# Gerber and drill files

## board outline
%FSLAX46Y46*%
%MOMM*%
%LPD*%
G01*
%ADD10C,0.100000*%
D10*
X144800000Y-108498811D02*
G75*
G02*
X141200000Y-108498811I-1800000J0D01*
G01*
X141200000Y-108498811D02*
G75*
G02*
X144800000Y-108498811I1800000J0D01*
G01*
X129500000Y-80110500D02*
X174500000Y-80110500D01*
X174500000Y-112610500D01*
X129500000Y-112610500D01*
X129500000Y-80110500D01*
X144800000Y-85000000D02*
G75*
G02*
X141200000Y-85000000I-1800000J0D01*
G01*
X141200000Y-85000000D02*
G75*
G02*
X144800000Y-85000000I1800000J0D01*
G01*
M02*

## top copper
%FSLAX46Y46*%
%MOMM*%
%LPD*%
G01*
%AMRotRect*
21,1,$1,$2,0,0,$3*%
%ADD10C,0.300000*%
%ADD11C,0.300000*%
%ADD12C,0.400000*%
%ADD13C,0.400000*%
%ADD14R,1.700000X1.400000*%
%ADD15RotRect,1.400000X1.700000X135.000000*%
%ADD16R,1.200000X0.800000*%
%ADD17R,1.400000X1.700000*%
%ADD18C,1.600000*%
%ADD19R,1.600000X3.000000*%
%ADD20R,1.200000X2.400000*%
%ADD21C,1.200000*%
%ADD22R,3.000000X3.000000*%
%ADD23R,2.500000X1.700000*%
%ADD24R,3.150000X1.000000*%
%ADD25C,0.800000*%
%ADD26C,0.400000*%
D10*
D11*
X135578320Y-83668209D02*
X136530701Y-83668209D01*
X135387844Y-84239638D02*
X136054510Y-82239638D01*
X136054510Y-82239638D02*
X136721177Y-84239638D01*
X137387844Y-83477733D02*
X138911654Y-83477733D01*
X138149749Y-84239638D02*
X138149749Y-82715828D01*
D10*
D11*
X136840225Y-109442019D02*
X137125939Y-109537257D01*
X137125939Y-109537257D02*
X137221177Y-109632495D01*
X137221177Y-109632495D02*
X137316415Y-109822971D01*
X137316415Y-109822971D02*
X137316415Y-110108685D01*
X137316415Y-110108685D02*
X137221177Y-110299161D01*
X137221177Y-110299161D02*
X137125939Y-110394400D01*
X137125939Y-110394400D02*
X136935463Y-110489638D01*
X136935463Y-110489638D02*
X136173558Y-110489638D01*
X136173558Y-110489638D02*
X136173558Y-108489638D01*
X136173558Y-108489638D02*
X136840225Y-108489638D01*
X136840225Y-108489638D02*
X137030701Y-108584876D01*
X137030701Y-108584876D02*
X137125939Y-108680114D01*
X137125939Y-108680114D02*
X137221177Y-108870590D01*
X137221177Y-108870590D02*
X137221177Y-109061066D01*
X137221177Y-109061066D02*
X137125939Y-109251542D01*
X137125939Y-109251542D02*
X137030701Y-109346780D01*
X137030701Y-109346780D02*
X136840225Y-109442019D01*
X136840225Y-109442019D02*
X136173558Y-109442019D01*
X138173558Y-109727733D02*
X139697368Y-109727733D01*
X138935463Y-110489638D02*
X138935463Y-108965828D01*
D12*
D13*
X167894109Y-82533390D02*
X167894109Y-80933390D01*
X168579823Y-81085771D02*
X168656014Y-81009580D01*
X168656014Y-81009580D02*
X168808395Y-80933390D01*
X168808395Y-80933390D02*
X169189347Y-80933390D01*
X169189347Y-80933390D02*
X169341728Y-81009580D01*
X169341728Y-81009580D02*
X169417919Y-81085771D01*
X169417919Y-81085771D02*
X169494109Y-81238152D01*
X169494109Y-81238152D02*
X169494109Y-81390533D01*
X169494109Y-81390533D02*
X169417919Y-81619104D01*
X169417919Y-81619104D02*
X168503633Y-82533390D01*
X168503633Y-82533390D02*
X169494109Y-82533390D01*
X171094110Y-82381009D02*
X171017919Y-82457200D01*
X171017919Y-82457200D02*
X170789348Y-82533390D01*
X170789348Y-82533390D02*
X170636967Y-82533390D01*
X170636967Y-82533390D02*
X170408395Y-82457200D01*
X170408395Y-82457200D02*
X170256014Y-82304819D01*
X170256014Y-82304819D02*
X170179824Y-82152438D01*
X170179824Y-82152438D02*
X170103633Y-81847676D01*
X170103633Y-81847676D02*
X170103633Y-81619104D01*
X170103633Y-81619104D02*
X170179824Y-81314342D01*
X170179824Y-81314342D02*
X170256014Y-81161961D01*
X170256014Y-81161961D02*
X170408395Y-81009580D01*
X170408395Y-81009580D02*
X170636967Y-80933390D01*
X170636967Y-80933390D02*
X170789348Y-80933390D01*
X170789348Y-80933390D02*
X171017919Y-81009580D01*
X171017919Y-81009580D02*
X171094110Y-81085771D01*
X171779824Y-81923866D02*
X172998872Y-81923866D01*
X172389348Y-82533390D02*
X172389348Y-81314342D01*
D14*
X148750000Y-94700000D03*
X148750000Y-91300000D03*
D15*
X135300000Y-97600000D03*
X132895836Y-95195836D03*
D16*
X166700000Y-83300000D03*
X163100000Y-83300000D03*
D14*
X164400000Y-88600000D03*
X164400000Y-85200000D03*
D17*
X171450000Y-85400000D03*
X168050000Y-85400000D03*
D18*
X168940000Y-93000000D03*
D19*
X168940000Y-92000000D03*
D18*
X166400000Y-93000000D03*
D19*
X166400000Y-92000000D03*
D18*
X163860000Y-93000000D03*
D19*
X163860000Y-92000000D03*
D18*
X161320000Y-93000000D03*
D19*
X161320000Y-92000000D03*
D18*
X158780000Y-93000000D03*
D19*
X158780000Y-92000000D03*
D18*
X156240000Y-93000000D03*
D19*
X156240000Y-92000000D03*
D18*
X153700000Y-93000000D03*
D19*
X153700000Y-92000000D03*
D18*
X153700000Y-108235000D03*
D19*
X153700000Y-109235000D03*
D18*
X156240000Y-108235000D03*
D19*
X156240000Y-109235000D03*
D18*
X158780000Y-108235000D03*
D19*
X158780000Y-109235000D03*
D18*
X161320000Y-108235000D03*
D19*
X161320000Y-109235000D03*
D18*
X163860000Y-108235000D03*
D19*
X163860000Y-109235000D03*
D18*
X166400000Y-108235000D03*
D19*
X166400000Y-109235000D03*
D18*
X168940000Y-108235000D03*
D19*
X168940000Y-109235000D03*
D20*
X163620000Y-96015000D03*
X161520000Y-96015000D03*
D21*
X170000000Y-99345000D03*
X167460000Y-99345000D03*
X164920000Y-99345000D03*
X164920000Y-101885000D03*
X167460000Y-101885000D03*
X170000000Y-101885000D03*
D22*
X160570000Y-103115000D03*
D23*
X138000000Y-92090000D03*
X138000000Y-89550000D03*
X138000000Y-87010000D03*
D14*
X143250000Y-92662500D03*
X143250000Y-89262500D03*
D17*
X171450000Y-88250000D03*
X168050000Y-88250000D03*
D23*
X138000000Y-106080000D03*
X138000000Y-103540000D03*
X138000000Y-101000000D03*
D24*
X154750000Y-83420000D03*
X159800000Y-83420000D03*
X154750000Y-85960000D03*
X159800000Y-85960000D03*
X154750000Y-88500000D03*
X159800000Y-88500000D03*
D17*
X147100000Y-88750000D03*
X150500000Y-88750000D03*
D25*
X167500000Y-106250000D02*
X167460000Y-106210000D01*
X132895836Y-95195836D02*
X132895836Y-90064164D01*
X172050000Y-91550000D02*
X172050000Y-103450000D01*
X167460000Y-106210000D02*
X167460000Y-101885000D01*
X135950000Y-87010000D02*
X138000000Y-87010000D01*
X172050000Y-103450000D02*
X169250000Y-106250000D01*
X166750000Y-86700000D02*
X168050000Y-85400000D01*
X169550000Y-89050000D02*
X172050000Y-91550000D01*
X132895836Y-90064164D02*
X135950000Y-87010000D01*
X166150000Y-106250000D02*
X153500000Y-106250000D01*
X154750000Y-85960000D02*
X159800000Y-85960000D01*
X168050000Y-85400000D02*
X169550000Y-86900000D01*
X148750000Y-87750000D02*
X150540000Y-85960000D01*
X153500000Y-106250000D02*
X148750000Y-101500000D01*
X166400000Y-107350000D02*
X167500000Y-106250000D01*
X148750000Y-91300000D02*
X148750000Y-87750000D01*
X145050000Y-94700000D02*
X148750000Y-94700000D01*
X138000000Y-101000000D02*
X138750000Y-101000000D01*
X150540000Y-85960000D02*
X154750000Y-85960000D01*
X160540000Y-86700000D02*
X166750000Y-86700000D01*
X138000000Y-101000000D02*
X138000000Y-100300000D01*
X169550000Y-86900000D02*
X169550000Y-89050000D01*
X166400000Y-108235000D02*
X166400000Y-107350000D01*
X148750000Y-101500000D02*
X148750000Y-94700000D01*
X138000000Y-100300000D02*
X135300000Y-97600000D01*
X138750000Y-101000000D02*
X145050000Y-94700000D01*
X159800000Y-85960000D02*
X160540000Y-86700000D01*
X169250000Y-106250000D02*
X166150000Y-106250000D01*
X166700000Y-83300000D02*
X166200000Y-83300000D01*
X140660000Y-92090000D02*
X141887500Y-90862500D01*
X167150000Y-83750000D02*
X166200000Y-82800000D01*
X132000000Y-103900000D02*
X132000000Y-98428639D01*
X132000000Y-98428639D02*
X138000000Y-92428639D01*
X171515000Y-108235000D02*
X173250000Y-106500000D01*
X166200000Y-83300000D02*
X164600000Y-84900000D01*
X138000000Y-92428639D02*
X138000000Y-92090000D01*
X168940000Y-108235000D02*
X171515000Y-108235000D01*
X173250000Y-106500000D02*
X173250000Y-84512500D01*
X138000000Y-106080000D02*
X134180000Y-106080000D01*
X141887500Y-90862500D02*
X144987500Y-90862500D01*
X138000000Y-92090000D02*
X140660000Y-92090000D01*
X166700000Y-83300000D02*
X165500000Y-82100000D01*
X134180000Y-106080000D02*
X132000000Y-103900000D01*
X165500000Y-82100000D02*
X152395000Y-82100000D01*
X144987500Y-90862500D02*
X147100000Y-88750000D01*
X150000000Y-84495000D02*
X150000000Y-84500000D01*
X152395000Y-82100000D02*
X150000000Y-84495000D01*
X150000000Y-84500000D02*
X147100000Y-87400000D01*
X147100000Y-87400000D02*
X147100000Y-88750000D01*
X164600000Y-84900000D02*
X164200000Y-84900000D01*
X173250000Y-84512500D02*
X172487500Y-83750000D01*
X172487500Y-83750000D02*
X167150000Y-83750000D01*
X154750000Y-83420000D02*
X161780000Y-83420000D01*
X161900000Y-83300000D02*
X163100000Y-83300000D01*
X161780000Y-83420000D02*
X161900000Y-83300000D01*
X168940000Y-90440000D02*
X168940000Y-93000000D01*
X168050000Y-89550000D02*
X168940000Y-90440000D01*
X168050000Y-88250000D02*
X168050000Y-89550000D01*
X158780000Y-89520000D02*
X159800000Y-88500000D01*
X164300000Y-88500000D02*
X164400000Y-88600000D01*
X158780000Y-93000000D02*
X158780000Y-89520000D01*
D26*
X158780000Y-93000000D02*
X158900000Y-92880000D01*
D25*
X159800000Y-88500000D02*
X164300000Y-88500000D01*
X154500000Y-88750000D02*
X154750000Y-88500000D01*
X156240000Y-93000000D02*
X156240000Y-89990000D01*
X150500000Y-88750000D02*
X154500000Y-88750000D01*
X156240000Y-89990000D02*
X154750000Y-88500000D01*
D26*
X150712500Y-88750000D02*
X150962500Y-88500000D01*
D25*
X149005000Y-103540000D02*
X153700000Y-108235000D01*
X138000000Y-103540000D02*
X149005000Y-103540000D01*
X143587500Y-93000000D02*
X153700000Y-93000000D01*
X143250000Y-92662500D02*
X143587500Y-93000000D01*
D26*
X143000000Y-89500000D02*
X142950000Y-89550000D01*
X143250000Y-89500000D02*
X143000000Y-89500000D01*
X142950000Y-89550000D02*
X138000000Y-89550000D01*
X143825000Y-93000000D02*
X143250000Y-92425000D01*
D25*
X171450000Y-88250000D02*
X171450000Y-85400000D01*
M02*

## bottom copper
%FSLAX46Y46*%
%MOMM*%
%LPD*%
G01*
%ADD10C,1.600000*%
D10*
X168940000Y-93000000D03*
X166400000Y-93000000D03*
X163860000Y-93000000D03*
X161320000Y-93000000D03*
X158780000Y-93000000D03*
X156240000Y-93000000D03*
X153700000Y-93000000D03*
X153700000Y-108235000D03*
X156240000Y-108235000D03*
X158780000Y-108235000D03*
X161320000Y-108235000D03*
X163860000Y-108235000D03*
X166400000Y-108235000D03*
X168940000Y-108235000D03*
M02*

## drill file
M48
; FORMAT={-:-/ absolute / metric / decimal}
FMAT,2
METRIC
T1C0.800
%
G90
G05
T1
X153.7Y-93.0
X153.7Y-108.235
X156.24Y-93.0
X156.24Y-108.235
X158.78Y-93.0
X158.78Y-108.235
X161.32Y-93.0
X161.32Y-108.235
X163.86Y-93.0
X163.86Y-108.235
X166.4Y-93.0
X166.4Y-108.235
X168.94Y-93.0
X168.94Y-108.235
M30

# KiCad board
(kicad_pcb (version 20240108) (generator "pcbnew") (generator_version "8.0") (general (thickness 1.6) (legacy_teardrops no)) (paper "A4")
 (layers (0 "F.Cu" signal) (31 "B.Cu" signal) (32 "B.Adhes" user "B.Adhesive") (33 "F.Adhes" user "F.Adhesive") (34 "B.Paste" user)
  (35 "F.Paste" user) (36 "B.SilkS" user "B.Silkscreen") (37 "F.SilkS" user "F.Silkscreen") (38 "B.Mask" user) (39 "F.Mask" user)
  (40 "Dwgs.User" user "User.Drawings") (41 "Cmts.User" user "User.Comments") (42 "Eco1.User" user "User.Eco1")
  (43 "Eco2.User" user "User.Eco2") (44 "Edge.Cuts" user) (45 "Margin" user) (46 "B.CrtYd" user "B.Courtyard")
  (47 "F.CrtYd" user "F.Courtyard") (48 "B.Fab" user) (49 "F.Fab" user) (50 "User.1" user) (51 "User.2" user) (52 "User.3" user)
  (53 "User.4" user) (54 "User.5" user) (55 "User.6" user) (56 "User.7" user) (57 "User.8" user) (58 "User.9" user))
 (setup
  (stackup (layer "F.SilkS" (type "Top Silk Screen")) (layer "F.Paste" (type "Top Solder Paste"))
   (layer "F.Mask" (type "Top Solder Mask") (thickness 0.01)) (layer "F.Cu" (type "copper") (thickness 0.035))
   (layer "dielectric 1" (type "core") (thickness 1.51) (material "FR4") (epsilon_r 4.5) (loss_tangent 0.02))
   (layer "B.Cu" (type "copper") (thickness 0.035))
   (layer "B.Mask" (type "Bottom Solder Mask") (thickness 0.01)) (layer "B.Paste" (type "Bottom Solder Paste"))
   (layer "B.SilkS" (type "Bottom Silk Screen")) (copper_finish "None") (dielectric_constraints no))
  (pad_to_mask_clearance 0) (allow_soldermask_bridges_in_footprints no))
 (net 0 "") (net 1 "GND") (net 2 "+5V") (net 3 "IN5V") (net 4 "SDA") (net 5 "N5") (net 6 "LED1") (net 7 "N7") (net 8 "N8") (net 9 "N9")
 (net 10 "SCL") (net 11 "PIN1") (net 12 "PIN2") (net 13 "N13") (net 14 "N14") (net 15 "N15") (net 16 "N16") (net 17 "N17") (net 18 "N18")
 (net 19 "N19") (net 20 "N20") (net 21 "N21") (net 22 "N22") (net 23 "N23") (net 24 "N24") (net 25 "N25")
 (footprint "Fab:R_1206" (layer "F.Cu") (at 148.75 93 90)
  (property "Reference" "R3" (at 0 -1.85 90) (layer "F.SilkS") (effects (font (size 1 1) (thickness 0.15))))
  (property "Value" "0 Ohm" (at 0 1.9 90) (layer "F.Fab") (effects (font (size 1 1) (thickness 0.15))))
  (pad "1" smd rect (at -1.7 0 90) (size 1.4 1.7) (layers "F.Cu" "F.Paste" "F.Mask") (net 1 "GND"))
  (pad "2" smd rect (at 1.7 0 90) (size 1.4 1.7) (layers "F.Cu" "F.Paste" "F.Mask") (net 1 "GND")))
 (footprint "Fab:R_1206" (layer "F.Cu") (at 134.097918 96.397918 135)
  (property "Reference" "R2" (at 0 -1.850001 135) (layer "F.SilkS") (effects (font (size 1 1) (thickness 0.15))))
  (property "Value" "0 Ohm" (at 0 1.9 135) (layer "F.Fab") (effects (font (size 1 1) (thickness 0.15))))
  (pad "1" smd rect (at -1.700001 0 135) (size 1.4 1.7) (layers "F.Cu" "F.Paste" "F.Mask") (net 1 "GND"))
  (pad "2" smd rect (at 1.700001 0 135) (size 1.4 1.7) (layers "F.Cu" "F.Paste" "F.Mask") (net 1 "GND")))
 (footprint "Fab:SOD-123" (layer "F.Cu") (at 164.9 83.3 180)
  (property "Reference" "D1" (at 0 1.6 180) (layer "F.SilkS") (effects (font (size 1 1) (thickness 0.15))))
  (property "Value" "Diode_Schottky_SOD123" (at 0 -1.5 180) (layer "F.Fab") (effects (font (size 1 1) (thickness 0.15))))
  (pad "1" smd rect (at -1.8 0 180) (size 1.2 0.8) (layers "F.Cu" "F.Paste" "F.Mask") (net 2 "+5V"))
  (pad "2" smd rect (at 1.8 0 180) (size 1.2 0.8) (layers "F.Cu" "F.Paste" "F.Mask") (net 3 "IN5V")))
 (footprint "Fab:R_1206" (layer "F.Cu") (at 164.4 86.9 90)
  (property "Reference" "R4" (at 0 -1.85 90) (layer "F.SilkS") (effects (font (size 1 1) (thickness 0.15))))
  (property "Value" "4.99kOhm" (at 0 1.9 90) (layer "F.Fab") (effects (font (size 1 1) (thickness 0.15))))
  (pad "1" smd rect (at -1.7 0 90) (size 1.4 1.7) (layers "F.Cu" "F.Paste" "F.Mask") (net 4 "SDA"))
  (pad "2" smd rect (at 1.7 0 90) (size 1.4 1.7) (layers "F.Cu" "F.Paste" "F.Mask") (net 2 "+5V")))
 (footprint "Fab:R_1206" (layer "F.Cu") (at 169.75 85.4 180)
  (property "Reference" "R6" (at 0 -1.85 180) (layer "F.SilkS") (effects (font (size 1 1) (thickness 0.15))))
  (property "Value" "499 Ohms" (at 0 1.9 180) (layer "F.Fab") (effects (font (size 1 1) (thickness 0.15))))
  (pad "1" smd rect (at -1.7 0 180) (size 1.4 1.7) (layers "F.Cu" "F.Paste" "F.Mask") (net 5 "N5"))
  (pad "2" smd rect (at 1.7 0 180) (size 1.4 1.7) (layers "F.Cu" "F.Paste" "F.Mask") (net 1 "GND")))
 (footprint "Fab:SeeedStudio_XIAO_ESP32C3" (layer "F.Cu") (at 161.32 100.615 -90)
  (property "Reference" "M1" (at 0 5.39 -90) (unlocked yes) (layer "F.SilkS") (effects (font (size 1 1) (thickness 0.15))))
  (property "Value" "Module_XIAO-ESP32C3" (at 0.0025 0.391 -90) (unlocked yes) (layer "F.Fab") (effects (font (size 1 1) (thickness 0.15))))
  (pad "1" thru_hole circle (at -7.615 -7.62 270) (size 1.6 1.6) (drill 0.8) (layers "*.Cu" "*.Mask") (remove_unused_layers yes)
   (keep_end_layers yes) (zone_layer_connections) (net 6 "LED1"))
  (pad "1" smd rect (at -7.615 -7.62 270) (size 3 1.6) (drill (offset -1 0)) (layers "F.Cu" "F.Paste" "F.Mask") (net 6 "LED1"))
  (pad "2" thru_hole circle (at -7.615 -5.08 270) (size 1.6 1.6) (drill 0.8) (layers "*.Cu" "*.Mask") (remove_unused_layers yes)
   (keep_end_layers yes) (zone_layer_connections) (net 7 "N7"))
  (pad "2" smd rect (at -7.615 -5.08 270) (size 3 1.6) (drill (offset -1 0)) (layers "F.Cu" "F.Paste" "F.Mask") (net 7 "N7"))
  (pad "3" thru_hole circle (at -7.615 -2.54 270) (size 1.6 1.6) (drill 0.8) (layers "*.Cu" "*.Mask") (remove_unused_layers yes)
   (keep_end_layers yes) (zone_layer_connections) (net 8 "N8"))
  (pad "3" smd rect (at -7.615 -2.54 270) (size 3 1.6) (drill (offset -1 0)) (layers "F.Cu" "F.Paste" "F.Mask") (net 8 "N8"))
  (pad "4" thru_hole circle (at -7.615 0 270) (size 1.6 1.6) (drill 0.8) (layers "*.Cu" "*.Mask") (remove_unused_layers yes)
   (keep_end_layers yes) (zone_layer_connections) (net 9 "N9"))
  (pad "4" smd rect (at -7.615 0 270) (size 3 1.6) (drill (offset -1 0)) (layers "F.Cu" "F.Paste" "F.Mask") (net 9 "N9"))
  (pad "5" thru_hole circle (at -7.615 2.54 270) (size 1.6 1.6) (drill 0.8) (layers "*.Cu" "*.Mask") (remove_unused_layers yes)
   (keep_end_layers yes) (zone_layer_connections) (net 4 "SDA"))
  (pad "5" smd rect (at -7.615 2.54 270) (size 3 1.6) (drill (offset -1 0)) (layers "F.Cu" "F.Paste" "F.Mask") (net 4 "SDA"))
  (pad "6" thru_hole circle (at -7.615 5.08 270) (size 1.6 1.6) (drill 0.8) (layers "*.Cu" "*.Mask") (remove_unused_layers yes)
   (keep_end_layers yes) (zone_layer_connections) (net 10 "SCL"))
  (pad "6" smd rect (at -7.615 5.08 270) (size 3 1.6) (drill (offset -1 0)) (layers "F.Cu" "F.Paste" "F.Mask") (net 10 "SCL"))
  (pad "7" thru_hole circle (at -7.615 7.62 270) (size 1.6 1.6) (drill 0.8) (layers "*.Cu" "*.Mask") (remove_unused_layers yes)
   (keep_end_layers yes) (zone_layer_connections) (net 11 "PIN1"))
  (pad "7" smd rect (at -7.615 7.62 270) (size 3 1.6) (drill (offset -1 0)) (layers "F.Cu" "F.Paste" "F.Mask") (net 11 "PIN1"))
  (pad "8" thru_hole circle (at 7.62 7.62 270) (size 1.6 1.6) (drill 0.8) (layers "*.Cu" "*.Mask") (remove_unused_layers yes)
   (keep_end_layers yes) (zone_layer_connections) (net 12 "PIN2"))
  (pad "8" smd rect (at 7.62 7.62 270) (size 3 1.6) (drill (offset 1 0)) (layers "F.Cu" "F.Paste" "F.Mask") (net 12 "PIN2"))
  (pad "9" thru_hole circle (at 7.62 5.08 270) (size 1.6 1.6) (drill 0.8) (layers "*.Cu" "*.Mask") (remove_unused_layers yes)
   (keep_end_layers yes) (zone_layer_connections) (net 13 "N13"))
  (pad "9" smd rect (at 7.62 5.08 270) (size 3 1.6) (drill (offset 1 0)) (layers "F.Cu" "F.Paste" "F.Mask") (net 13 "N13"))
  (pad "10" thru_hole circle (at 7.62 2.54 270) (size 1.6 1.6) (drill 0.8) (layers "*.Cu" "*.Mask") (remove_unused_layers yes)
   (keep_end_layers yes) (zone_layer_connections) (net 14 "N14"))
  (pad "10" smd rect (at 7.62 2.54 270) (size 3 1.6) (drill (offset 1 0)) (layers "F.Cu" "F.Paste" "F.Mask") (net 14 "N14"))
  (pad "11" thru_hole circle (at 7.62 0 270) (size 1.6 1.6) (drill 0.8) (layers "*.Cu" "*.Mask") (remove_unused_layers yes)
   (keep_end_layers yes) (zone_layer_connections) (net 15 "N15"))
  (pad "11" smd rect (at 7.62 0 270) (size 3 1.6) (drill (offset 1 0)) (layers "F.Cu" "F.Paste" "F.Mask") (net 15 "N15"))
  (pad "12" thru_hole circle (at 7.62 -2.54 270) (size 1.6 1.6) (drill 0.8) (layers "*.Cu" "*.Mask") (remove_unused_layers yes)
   (keep_end_layers yes) (zone_layer_connections) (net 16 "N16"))
  (pad "12" smd rect (at 7.62 -2.54 270) (size 3 1.6) (drill (offset 1 0)) (layers "F.Cu" "F.Paste" "F.Mask") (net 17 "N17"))
  (pad "13" thru_hole circle (at 7.62 -5.08 270) (size 1.6 1.6) (drill 0.8) (layers "*.Cu" "*.Mask") (remove_unused_layers yes)
   (keep_end_layers yes) (zone_layer_connections) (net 1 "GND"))
  (pad "13" smd rect (at 7.62 -5.08 270) (size 3 1.6) (drill (offset 1 0)) (layers "F.Cu" "F.Paste" "F.Mask") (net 1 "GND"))
  (pad "14" thru_hole circle (at 7.62 -7.62 270) (size 1.6 1.6) (drill 0.8) (layers "*.Cu" "*.Mask") (remove_unused_layers yes)
   (keep_end_layers yes) (zone_layer_connections) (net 2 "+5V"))
  (pad "14" smd rect (at 7.62 -7.62 270) (size 3 1.6) (drill (offset 1 0)) (layers "F.Cu" "F.Paste" "F.Mask") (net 2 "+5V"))
  (pad "15" smd rect (at -4.6 -2.3 270) (size 2.4 1.2) (layers "F.Cu" "F.Paste" "F.Mask") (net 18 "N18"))
  (pad "16" smd rect (at -4.6 -0.2 270) (size 2.4 1.2) (layers "F.Cu" "F.Paste" "F.Mask") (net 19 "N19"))
  (pad "17" smd circle (at -1.27 -8.68 270) (size 1.2 1.2) (layers "F.Cu" "F.Paste" "F.Mask") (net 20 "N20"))
  (pad "18" smd circle (at -1.27 -6.14 270) (size 1.2 1.2) (layers "F.Cu" "F.Paste" "F.Mask") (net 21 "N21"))
  (pad "19" smd circle (at -1.27 -3.6 270) (size 1.2 1.2) (layers "F.Cu" "F.Paste" "F.Mask") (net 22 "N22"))
  (pad "20" smd circle (at 1.27 -3.6 270) (size 1.2 1.2) (layers "F.Cu" "F.Paste" "F.Mask") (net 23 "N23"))
  (pad "21" smd circle (at 1.27 -6.14 270) (size 1.2 1.2) (layers "F.Cu" "F.Paste" "F.Mask") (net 1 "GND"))
  (pad "22" smd circle (at 1.27 -8.68 270) (size 1.2 1.2) (layers "F.Cu" "F.Paste" "F.Mask") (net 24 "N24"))
  (pad "23" smd rect (at 2.5 0.75 270) (size 3 3) (layers "F.Cu" "F.Paste" "F.Mask") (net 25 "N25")))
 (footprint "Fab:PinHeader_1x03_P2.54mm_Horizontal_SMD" (layer "F.Cu") (at 138 92.09 180)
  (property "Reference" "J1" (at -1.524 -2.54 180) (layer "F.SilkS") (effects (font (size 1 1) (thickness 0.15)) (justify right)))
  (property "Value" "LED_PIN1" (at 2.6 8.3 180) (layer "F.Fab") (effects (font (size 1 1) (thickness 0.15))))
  (pad "1" smd rect (at 0 0 180) (size 2.5 1.7) (layers "F.Cu" "F.Paste" "F.Mask") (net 2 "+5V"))
  (pad "2" smd rect (at 0 2.54 180) (size 2.5 1.7) (layers "F.Cu" "F.Paste" "F.Mask") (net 11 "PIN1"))
  (pad "3" smd rect (at 0 5.08 180) (size 2.5 1.7) (layers "F.Cu" "F.Paste" "F.Mask") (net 1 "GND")))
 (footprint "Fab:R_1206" (layer "F.Cu") (at 143.25 90.9625 90)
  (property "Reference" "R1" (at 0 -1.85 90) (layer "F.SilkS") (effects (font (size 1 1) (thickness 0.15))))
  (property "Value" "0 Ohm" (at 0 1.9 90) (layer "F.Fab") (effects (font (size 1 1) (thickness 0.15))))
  (pad "1" smd rect (at -1.7 0 90) (size 1.4 1.7) (layers "F.Cu" "F.Paste" "F.Mask") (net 11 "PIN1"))
  (pad "2" smd rect (at 1.7 0 90) (size 1.4 1.7) (layers "F.Cu" "F.Paste" "F.Mask") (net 11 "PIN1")))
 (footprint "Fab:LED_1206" (layer "F.Cu") (at 169.75 88.25 180)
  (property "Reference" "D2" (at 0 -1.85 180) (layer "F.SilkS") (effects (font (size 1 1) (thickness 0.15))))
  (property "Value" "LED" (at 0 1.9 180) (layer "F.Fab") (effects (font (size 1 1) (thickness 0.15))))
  (pad "1" smd rect (at -1.7 0 180) (size 1.4 1.7) (layers "F.Cu" "F.Paste" "F.Mask") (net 5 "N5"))
  (pad "2" smd rect (at 1.7 0 180) (size 1.4 1.7) (layers "F.Cu" "F.Paste" "F.Mask") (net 6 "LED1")))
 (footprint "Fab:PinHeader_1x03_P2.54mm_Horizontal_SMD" (layer "F.Cu") (at 138 106.08 180)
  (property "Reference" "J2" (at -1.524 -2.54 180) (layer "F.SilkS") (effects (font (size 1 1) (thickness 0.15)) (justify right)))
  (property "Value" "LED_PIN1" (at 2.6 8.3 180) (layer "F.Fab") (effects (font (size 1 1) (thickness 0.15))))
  (pad "1" smd rect (at 0 0 180) (size 2.5 1.7) (layers "F.Cu" "F.Paste" "F.Mask") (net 2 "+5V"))
  (pad "2" smd rect (at 0 2.54 180) (size 2.5 1.7) (layers "F.Cu" "F.Paste" "F.Mask") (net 12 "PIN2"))
  (pad "3" smd rect (at 0 5.08 180) (size 2.5 1.7) (layers "F.Cu" "F.Paste" "F.Mask") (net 1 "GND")))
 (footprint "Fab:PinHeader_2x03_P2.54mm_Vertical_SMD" (layer "F.Cu") (at 157.275 85.96)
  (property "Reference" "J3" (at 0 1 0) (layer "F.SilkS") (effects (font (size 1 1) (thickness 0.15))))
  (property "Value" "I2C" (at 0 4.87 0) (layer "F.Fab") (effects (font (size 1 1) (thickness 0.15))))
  (pad "1" smd rect (at -2.525 -2.54) (size 3.15 1) (layers "F.Cu" "F.Paste" "F.Mask") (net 3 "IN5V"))
  (pad "2" smd rect (at 2.525 -2.54) (size 3.15 1) (layers "F.Cu" "F.Paste" "F.Mask") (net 3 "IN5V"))
  (pad "3" smd rect (at -2.525 0) (size 3.15 1) (layers "F.Cu" "F.Paste" "F.Mask") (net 1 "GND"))
  (pad "4" smd rect (at 2.525 0) (size 3.15 1) (layers "F.Cu" "F.Paste" "F.Mask") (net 1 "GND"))
  (pad "5" smd rect (at -2.525 2.54) (size 3.15 1) (layers "F.Cu" "F.Paste" "F.Mask") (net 10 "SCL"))
  (pad "6" smd rect (at 2.525 2.54) (size 3.15 1) (layers "F.Cu" "F.Paste" "F.Mask") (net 4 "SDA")))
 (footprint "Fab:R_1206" (layer "F.Cu") (at 148.8 88.75)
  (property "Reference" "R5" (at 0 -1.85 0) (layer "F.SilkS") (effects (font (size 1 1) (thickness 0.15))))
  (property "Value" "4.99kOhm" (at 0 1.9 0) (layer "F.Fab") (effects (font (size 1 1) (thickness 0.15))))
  (pad "1" smd rect (at -1.7 0) (size 1.4 1.7) (layers "F.Cu" "F.Paste" "F.Mask") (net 2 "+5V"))
  (pad "2" smd rect (at 1.7 0) (size 1.4 1.7) (layers "F.Cu" "F.Paste" "F.Mask") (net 10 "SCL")))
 (gr_circle (center 143 108.498811) (end 144.8 108.498811) (stroke (width 0.1) (type default)) (fill none) (layer "Edge.Cuts"))
 (gr_rect (start 129.5 80.1105) (end 174.5 112.6105) (stroke (width 0.1) (type solid)) (fill none) (layer "Edge.Cuts"))
 (gr_circle (center 143 85) (end 144.8 85) (stroke (width 0.1) (type default)) (fill none) (layer "Edge.Cuts"))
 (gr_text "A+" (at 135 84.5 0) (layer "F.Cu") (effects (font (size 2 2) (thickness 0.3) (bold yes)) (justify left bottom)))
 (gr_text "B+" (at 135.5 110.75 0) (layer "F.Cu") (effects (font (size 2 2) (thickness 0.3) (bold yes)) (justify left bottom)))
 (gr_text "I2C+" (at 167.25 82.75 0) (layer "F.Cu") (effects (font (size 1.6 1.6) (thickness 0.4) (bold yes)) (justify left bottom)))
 (segment (start 167.5 106.25) (end 167.46 106.21) (width 0.8) (layer "F.Cu") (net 1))
 (segment (start 132.895836 95.195836) (end 132.895836 90.064164) (width 0.8) (layer "F.Cu") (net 1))
 (segment (start 172.05 91.55) (end 172.05 103.45) (width 0.8) (layer "F.Cu") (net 1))
 (segment (start 167.46 106.21) (end 167.46 101.885) (width 0.8) (layer "F.Cu") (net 1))
 (segment (start 135.95 87.01) (end 138 87.01) (width 0.8) (layer "F.Cu") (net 1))
 (segment (start 172.05 103.45) (end 169.25 106.25) (width 0.8) (layer "F.Cu") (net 1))
 (segment (start 166.75 86.7) (end 168.05 85.4) (width 0.8) (layer "F.Cu") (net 1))
 (segment (start 169.55 89.05) (end 172.05 91.55) (width 0.8) (layer "F.Cu") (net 1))
 (segment (start 132.895836 90.064164) (end 135.95 87.01) (width 0.8) (layer "F.Cu") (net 1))
 (segment (start 166.15 106.25) (end 153.5 106.25) (width 0.8) (layer "F.Cu") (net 1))
 (segment (start 154.75 85.96) (end 159.8 85.96) (width 0.8) (layer "F.Cu") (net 1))
 (segment (start 168.05 85.4) (end 169.55 86.9) (width 0.8) (layer "F.Cu") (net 1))
 (segment (start 148.75 87.75) (end 150.54 85.96) (width 0.8) (layer "F.Cu") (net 1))
 (segment (start 153.5 106.25) (end 148.75 101.5) (width 0.8) (layer "F.Cu") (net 1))
 (segment (start 166.4 107.35) (end 167.5 106.25) (width 0.8) (layer "F.Cu") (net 1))
 (segment (start 148.75 91.3) (end 148.75 87.75) (width 0.8) (layer "F.Cu") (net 1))
 (segment (start 145.05 94.7) (end 148.75 94.7) (width 0.8) (layer "F.Cu") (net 1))
 (segment (start 138 101) (end 138.75 101) (width 0.8) (layer "F.Cu") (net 1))
 (segment (start 150.54 85.96) (end 154.75 85.96) (width 0.8) (layer "F.Cu") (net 1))
 (segment (start 160.54 86.7) (end 166.75 86.7) (width 0.8) (layer "F.Cu") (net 1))
 (segment (start 138 101) (end 138 100.3) (width 0.8) (layer "F.Cu") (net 1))
 (segment (start 169.55 86.9) (end 169.55 89.05) (width 0.8) (layer "F.Cu") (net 1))
 (segment (start 166.4 108.235) (end 166.4 107.35) (width 0.8) (layer "F.Cu") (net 1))
 (segment (start 148.75 101.5) (end 148.75 94.7) (width 0.8) (layer "F.Cu") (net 1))
 (segment (start 138 100.3) (end 135.3 97.6) (width 0.8) (layer "F.Cu") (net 1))
 (segment (start 138.75 101) (end 145.05 94.7) (width 0.8) (layer "F.Cu") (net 1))
 (segment (start 159.8 85.96) (end 160.54 86.7) (width 0.8) (layer "F.Cu") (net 1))
 (segment (start 169.25 106.25) (end 166.15 106.25) (width 0.8) (layer "F.Cu") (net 1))
 (segment (start 166.7 83.3) (end 166.2 83.3) (width 0.8) (layer "F.Cu") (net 2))
 (segment (start 140.66 92.09) (end 141.8875 90.8625) (width 0.8) (layer "F.Cu") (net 2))
 (segment (start 167.15 83.75) (end 166.2 82.8) (width 0.8) (layer "F.Cu") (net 2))
 (segment (start 132 103.9) (end 132 98.428639) (width 0.8) (layer "F.Cu") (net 2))
 (segment (start 132 98.428639) (end 138 92.428639) (width 0.8) (layer "F.Cu") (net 2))
 (segment (start 171.515 108.235) (end 173.25 106.5) (width 0.8) (layer "F.Cu") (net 2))
 (segment (start 166.2 83.3) (end 164.6 84.9) (width 0.8) (layer "F.Cu") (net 2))
 (segment (start 138 92.428639) (end 138 92.09) (width 0.8) (layer "F.Cu") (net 2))
 (segment (start 168.94 108.235) (end 171.515 108.235) (width 0.8) (layer "F.Cu") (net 2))
 (segment (start 173.25 106.5) (end 173.25 84.5125) (width 0.8) (layer "F.Cu") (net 2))
 (segment (start 138 106.08) (end 134.18 106.08) (width 0.8) (layer "F.Cu") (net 2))
 (segment (start 141.8875 90.8625) (end 144.9875 90.8625) (width 0.8) (layer "F.Cu") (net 2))
 (segment (start 138 92.09) (end 140.66 92.09) (width 0.8) (layer "F.Cu") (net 2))
 (segment (start 166.7 83.3) (end 165.5 82.1) (width 0.8) (layer "F.Cu") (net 2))
 (segment (start 134.18 106.08) (end 132 103.9) (width 0.8) (layer "F.Cu") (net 2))
 (segment (start 165.5 82.1) (end 152.395 82.1) (width 0.8) (layer "F.Cu") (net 2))
 (segment (start 144.9875 90.8625) (end 147.1 88.75) (width 0.8) (layer "F.Cu") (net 2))
 (segment (start 150 84.495) (end 150 84.5) (width 0.8) (layer "F.Cu") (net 2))
 (segment (start 152.395 82.1) (end 150 84.495) (width 0.8) (layer "F.Cu") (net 2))
 (segment (start 150 84.5) (end 147.1 87.4) (width 0.8) (layer "F.Cu") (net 2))
 (segment (start 147.1 87.4) (end 147.1 88.75) (width 0.8) (layer "F.Cu") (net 2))
 (segment (start 164.6 84.9) (end 164.2 84.9) (width 0.8) (layer "F.Cu") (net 2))
 (segment (start 173.25 84.5125) (end 172.4875 83.75) (width 0.8) (layer "F.Cu") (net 2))
 (segment (start 172.4875 83.75) (end 167.15 83.75) (width 0.8) (layer "F.Cu") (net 2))
 (segment (start 154.75 83.42) (end 161.78 83.42) (width 0.8) (layer "F.Cu") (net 3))
 (segment (start 161.9 83.3) (end 163.1 83.3) (width 0.8) (layer "F.Cu") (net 3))
 (segment (start 161.78 83.42) (end 161.9 83.3) (width 0.8) (layer "F.Cu") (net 3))
 (segment (start 168.94 90.44) (end 168.94 93) (width 0.8) (layer "F.Cu") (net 6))
 (segment (start 168.05 89.55) (end 168.94 90.44) (width 0.8) (layer "F.Cu") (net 6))
 (segment (start 168.05 88.25) (end 168.05 89.55) (width 0.8) (layer "F.Cu") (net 6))
 (segment (start 158.78 89.52) (end 159.8 88.5) (width 0.8) (layer "F.Cu") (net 4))
 (segment (start 164.3 88.5) (end 164.4 88.6) (width 0.8) (layer "F.Cu") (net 4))
 (segment (start 158.78 93) (end 158.78 89.52) (width 0.8) (layer "F.Cu") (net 4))
 (segment (start 158.78 93) (end 158.9 92.88) (width 0.4) (layer "F.Cu") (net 4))
 (segment (start 159.8 88.5) (end 164.3 88.5) (width 0.8) (layer "F.Cu") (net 4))
 (segment (start 154.5 88.75) (end 154.75 88.5) (width 0.8) (layer "F.Cu") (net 10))
 (segment (start 156.24 93) (end 156.24 89.99) (width 0.8) (layer "F.Cu") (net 10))
 (segment (start 150.5 88.75) (end 154.5 88.75) (width 0.8) (layer "F.Cu") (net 10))
 (segment (start 156.24 89.99) (end 154.75 88.5) (width 0.8) (layer "F.Cu") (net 10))
 (segment (start 150.7125 88.75) (end 150.9625 88.5) (width 0.4) (layer "F.Cu") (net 10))
 (segment (start 149.005 103.54) (end 153.7 108.235) (width 0.8) (layer "F.Cu") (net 12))
 (segment (start 138 103.54) (end 149.005 103.54) (width 0.8) (layer "F.Cu") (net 12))
 (segment (start 143.5875 93) (end 153.7 93) (width 0.8) (layer "F.Cu") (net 11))
 (segment (start 143.25 92.6625) (end 143.5875 93) (width 0.8) (layer "F.Cu") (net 11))
 (segment (start 143 89.5) (end 142.95 89.55) (width 0.4) (layer "F.Cu") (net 11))
 (segment (start 143.25 89.5) (end 143 89.5) (width 0.4) (layer "F.Cu") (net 11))
 (segment (start 142.95 89.55) (end 138 89.55) (width 0.4) (layer "F.Cu") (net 11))
 (segment (start 143.825 93) (end 143.25 92.425) (width 0.4) (layer "F.Cu") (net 11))
 (segment (start 171.45 88.25) (end 171.45 85.4) (width 0.8) (layer "F.Cu") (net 5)))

